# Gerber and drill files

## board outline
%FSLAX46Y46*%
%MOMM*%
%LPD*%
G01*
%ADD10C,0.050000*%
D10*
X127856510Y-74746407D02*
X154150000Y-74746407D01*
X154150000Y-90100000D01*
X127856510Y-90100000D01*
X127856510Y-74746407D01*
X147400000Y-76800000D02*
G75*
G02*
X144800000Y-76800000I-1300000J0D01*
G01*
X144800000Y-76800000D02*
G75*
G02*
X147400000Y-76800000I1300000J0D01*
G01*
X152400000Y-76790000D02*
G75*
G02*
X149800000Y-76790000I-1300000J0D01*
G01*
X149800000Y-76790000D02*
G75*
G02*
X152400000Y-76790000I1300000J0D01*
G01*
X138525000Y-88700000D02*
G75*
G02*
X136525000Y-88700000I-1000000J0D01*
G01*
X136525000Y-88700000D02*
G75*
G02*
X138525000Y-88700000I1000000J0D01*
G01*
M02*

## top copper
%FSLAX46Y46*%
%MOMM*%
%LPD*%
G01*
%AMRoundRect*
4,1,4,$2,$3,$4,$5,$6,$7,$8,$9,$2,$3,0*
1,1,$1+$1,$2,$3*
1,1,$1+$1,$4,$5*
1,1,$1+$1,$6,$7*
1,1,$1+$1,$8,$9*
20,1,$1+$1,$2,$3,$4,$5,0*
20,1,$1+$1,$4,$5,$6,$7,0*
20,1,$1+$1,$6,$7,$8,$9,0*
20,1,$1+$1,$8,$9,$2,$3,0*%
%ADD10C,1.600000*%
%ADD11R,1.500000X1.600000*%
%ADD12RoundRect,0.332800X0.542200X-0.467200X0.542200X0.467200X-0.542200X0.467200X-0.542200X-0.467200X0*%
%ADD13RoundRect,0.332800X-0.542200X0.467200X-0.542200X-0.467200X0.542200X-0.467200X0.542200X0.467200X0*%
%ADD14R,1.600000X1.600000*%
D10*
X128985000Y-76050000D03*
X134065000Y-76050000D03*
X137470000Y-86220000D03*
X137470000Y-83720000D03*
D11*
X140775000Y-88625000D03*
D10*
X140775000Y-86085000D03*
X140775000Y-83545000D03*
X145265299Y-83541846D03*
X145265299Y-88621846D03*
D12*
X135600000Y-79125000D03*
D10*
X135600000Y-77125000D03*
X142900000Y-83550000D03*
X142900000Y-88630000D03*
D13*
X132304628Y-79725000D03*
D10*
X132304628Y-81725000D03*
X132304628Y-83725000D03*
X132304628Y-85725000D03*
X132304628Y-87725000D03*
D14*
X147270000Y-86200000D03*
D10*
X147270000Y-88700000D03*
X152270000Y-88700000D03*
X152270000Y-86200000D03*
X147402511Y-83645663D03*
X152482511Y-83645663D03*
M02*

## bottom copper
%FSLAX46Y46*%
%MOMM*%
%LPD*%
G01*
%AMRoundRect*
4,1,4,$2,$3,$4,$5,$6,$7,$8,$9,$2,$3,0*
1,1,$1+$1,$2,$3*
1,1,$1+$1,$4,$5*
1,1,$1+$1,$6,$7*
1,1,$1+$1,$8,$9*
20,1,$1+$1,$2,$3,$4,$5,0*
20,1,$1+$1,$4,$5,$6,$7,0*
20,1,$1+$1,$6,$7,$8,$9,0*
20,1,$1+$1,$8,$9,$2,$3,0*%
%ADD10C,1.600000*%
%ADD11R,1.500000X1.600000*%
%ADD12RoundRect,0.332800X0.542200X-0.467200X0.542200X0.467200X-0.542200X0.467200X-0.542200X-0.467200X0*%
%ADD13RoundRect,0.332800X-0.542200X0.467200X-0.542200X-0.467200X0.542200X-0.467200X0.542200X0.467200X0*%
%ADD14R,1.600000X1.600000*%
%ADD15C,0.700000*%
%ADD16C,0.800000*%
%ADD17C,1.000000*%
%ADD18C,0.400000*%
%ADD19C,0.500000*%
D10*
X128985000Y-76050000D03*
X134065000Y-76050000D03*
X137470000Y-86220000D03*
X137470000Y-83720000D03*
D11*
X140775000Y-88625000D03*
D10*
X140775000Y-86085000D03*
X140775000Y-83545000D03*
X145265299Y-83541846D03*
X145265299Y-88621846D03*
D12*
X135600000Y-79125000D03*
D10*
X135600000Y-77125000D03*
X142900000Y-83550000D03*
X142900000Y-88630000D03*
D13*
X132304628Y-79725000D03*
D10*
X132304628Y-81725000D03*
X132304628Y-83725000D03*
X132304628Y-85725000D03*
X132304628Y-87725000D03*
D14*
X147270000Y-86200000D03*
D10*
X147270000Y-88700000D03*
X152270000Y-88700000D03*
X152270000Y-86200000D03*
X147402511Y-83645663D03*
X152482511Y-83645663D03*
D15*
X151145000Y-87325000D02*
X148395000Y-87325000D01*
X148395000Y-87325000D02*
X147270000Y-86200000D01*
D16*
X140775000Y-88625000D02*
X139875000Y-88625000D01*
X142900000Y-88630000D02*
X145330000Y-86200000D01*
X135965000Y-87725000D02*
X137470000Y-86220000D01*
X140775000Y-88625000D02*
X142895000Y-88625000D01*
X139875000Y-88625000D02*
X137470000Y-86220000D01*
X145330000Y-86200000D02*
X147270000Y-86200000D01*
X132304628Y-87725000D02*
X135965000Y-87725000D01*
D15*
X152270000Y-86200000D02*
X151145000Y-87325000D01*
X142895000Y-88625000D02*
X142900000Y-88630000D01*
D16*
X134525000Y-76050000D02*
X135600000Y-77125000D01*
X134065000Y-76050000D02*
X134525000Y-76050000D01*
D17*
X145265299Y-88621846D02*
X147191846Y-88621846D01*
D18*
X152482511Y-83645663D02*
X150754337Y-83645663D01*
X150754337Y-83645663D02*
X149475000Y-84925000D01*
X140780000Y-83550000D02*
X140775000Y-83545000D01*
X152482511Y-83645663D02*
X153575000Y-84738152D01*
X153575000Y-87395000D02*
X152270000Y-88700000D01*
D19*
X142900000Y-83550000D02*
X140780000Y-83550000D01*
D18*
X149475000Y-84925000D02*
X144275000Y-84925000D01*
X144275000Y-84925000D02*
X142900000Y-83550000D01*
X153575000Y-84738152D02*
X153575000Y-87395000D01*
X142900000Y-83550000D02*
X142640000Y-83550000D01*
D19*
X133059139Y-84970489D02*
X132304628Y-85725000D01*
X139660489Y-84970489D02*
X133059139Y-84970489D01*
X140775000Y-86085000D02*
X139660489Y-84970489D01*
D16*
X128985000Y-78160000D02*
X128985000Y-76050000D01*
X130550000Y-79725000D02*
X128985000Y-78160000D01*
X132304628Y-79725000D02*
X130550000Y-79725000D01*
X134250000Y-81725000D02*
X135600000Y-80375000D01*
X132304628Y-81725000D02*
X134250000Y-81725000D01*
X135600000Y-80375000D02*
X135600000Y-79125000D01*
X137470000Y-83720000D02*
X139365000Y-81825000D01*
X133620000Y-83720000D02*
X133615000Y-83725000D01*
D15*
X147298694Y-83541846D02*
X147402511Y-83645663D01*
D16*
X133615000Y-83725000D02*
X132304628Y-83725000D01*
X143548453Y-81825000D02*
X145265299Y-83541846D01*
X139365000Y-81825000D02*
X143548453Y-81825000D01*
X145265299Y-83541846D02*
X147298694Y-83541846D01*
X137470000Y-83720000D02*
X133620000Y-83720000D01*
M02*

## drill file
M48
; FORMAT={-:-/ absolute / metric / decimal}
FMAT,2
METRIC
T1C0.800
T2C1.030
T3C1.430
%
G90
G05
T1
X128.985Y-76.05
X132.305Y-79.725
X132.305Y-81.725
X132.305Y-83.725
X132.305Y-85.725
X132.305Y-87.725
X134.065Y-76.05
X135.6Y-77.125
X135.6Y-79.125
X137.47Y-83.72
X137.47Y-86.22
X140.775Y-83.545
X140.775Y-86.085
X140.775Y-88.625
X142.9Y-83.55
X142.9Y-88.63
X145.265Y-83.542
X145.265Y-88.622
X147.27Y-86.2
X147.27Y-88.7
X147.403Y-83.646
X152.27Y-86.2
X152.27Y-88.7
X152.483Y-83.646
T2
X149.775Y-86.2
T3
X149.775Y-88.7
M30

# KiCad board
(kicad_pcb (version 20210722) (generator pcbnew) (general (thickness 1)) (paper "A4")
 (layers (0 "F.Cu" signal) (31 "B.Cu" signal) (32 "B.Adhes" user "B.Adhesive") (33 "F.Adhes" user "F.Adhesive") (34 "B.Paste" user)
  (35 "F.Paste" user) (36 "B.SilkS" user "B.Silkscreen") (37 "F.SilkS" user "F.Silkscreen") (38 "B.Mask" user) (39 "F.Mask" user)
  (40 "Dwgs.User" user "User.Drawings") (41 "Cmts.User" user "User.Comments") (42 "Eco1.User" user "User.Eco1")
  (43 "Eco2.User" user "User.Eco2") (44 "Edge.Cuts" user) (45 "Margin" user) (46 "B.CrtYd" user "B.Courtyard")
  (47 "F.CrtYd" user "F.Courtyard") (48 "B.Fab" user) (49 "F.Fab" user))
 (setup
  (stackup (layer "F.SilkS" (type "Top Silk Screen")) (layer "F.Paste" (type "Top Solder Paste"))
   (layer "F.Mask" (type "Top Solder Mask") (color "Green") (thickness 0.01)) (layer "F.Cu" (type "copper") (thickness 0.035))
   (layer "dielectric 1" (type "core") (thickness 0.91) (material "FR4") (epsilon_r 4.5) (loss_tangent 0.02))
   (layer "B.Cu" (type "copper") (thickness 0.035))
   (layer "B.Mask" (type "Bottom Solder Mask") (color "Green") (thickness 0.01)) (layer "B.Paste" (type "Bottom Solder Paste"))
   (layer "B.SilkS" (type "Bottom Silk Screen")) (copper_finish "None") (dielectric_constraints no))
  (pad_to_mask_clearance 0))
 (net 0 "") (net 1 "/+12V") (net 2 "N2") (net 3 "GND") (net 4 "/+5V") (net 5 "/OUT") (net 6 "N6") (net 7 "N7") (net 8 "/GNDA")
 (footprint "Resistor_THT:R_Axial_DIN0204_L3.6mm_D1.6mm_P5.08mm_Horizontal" (layer "F.Cu") (at 128.985 76.05)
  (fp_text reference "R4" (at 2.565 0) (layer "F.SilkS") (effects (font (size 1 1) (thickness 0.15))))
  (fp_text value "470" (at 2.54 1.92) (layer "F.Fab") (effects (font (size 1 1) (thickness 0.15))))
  (pad "1" thru_hole circle locked (at 0 0) (size 1.6 1.6) (drill 0.8) (layers *.Cu *.Mask) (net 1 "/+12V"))
  (pad "2" thru_hole circle locked (at 5.08 0) (size 1.6 1.6) (drill 0.8) (layers *.Cu *.Mask) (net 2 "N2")))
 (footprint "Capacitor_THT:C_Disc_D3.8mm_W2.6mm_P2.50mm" (layer "F.Cu") (at 137.47 86.22 90)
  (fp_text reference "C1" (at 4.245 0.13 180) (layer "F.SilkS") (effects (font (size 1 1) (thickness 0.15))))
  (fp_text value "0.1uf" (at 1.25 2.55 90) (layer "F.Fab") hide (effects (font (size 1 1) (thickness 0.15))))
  (pad "1" thru_hole circle locked (at 0 0 90) (size 1.6 1.6) (drill 0.8) (layers *.Cu *.Mask) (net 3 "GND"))
  (pad "2" thru_hole circle locked (at 2.5 0 90) (size 1.6 1.6) (drill 0.8) (layers *.Cu *.Mask) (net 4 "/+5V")))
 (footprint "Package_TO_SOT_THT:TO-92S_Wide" (layer "F.Cu") (at 140.775 88.625 90)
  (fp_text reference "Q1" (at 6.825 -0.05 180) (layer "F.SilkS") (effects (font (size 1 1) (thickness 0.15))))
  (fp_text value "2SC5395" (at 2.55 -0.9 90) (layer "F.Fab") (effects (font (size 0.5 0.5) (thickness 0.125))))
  (pad "1" thru_hole rect locked (at 0 0 90) (size 1.6 1.5) (drill 0.8) (layers *.Cu *.Mask) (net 3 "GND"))
  (pad "2" thru_hole circle locked (at 2.54 0 90) (size 1.6 1.6) (drill 0.8) (layers *.Cu *.Mask) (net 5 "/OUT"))
  (pad "3" thru_hole circle locked (at 5.08 0 90) (size 1.6 1.6) (drill 0.8) (layers *.Cu *.Mask) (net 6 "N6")))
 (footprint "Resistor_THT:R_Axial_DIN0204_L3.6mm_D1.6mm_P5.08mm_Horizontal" (layer "F.Cu") (at 145.265299 83.541846 -90)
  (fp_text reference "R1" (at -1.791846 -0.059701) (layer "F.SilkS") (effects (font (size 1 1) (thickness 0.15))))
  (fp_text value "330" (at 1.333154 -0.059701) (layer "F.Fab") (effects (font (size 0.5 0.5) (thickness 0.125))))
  (pad "1" thru_hole circle locked (at 0 0 270) (size 1.6 1.6) (drill 0.8) (layers *.Cu *.Mask) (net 4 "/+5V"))
  (pad "2" thru_hole circle locked (at 5.08 0 270) (size 1.6 1.6) (drill 0.8) (layers *.Cu *.Mask) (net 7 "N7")))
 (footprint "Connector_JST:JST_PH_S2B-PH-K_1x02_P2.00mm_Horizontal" (layer "F.Cu") (at 135.6 79.125 90)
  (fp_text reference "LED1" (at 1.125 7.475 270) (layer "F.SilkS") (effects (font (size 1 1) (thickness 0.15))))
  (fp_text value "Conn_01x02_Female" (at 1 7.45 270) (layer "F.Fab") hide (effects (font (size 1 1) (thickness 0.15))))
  (pad "1" thru_hole roundrect locked (at 0 0 90) (size 1.6 1.75) (drill 0.8) (layers *.Cu *.Mask) (roundrect_rratio 0.208) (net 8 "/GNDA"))
  (pad "2" thru_hole circle locked (at 2 0 90) (size 1.6 1.6) (drill 0.8) (layers *.Cu *.Mask) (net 2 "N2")))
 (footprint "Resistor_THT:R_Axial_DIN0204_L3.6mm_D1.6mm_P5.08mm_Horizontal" (layer "F.Cu") (at 142.9 83.55 -90)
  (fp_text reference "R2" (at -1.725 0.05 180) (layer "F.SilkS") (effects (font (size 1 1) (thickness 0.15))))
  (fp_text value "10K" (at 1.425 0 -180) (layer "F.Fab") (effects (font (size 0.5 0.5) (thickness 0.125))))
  (pad "1" thru_hole circle locked (at 0 0 270) (size 1.6 1.6) (drill 0.8) (layers *.Cu *.Mask) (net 6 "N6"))
  (pad "2" thru_hole circle locked (at 5.08 0 270) (size 1.6 1.6) (drill 0.8) (layers *.Cu *.Mask) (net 3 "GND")))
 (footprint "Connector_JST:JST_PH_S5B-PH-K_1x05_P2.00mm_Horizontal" (layer "F.Cu") (at 132.304628 79.725 -90)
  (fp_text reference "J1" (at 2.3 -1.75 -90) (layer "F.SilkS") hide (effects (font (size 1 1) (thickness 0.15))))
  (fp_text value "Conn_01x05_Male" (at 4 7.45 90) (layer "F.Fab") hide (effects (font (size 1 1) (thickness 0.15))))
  (pad "1" thru_hole roundrect locked (at 0 0 270) (size 1.6 1.75) (drill 0.8) (layers *.Cu *.Mask) (roundrect_rratio 0.208) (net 1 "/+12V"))
  (pad "2" thru_hole circle locked (at 2 0 270) (size 1.6 1.6) (drill 0.8) (layers *.Cu *.Mask) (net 8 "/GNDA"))
  (pad "3" thru_hole circle locked (at 4 0 270) (size 1.6 1.6) (drill 0.8) (layers *.Cu *.Mask) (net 4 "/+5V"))
  (pad "4" thru_hole circle locked (at 6 0 270) (size 1.6 1.6) (drill 0.8) (layers *.Cu *.Mask) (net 5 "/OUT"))
  (pad "5" thru_hole circle locked (at 8 0 270) (size 1.6 1.6) (drill 0.8) (layers *.Cu *.Mask) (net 3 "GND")))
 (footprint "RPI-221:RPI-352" (layer "F.Cu") (at 146.5 89.6)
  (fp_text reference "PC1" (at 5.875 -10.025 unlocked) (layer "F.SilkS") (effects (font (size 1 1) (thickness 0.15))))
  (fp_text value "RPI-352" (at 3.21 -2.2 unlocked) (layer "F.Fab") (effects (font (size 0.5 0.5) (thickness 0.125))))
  (pad "" np_thru_hole circle locked (at 3.275 -3.4) (size 1.03 1.03) (drill 1.03) (layers *.Mask))
  (pad "" np_thru_hole circle locked (at 3.275 -0.9) (size 1.43 1.43) (drill 1.43) (layers *.Mask))
  (pad "1" thru_hole rect locked (at 0.77 -3.4) (size 1.6 1.6) (drill oval 0.8) (layers *.Cu *.Mask) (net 3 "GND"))
  (pad "2" thru_hole circle locked (at 0.77 -0.9) (size 1.6 1.6) (drill oval 0.8) (layers *.Cu *.Mask) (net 7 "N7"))
  (pad "3" thru_hole circle locked (at 5.77 -0.9) (size 1.6 1.6) (drill oval 0.8) (layers *.Cu *.Mask) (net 6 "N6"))
  (pad "4" thru_hole circle locked (at 5.77 -3.4) (size 1.6 1.6) (drill oval 0.8) (layers *.Cu *.Mask) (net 3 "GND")))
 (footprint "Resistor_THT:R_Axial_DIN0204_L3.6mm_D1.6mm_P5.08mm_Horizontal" (layer "F.Cu") (at 147.402511 83.645663)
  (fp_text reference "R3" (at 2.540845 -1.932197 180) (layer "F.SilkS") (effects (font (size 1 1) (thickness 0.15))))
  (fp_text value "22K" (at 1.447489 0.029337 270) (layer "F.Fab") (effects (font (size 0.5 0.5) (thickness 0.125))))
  (pad "1" thru_hole circle locked (at 0 0) (size 1.6 1.6) (drill 0.8) (layers *.Cu *.Mask) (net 4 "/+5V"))
  (pad "2" thru_hole circle locked (at 5.08 0) (size 1.6 1.6) (drill 0.8) (layers *.Cu *.Mask) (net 6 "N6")))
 (gr_rect (start 127.85651 74.746407) (end 154.15 90.1) (layer "Edge.Cuts") (width 0.05) (fill none))
 (gr_circle (center 146.1 76.8) (end 147.4 76.8) (layer "Edge.Cuts") (width 0.05) (fill none))
 (gr_circle (center 151.1 76.79) (end 152.4 76.79) (layer "Edge.Cuts") (width 0.05) (fill none))
 (gr_circle (center 137.525 88.7) (end 138.525 88.7) (layer "Edge.Cuts") (width 0.05) (fill none))
 (segment (start 151.145 87.325) (end 148.395 87.325) (width 0.7) (layer "B.Cu") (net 3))
 (segment (start 148.395 87.325) (end 147.27 86.2) (width 0.7) (layer "B.Cu") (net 3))
 (segment (start 140.775 88.625) (end 139.875 88.625) (width 0.8) (layer "B.Cu") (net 3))
 (segment (start 142.9 88.63) (end 145.33 86.2) (width 0.8) (layer "B.Cu") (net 3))
 (segment (start 135.965 87.725) (end 137.47 86.22) (width 0.8) (layer "B.Cu") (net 3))
 (segment (start 140.775 88.625) (end 142.895 88.625) (width 0.8) (layer "B.Cu") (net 3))
 (segment (start 139.875 88.625) (end 137.47 86.22) (width 0.8) (layer "B.Cu") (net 3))
 (segment (start 145.33 86.2) (end 147.27 86.2) (width 0.8) (layer "B.Cu") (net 3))
 (segment (start 132.304628 87.725) (end 135.965 87.725) (width 0.8) (layer "B.Cu") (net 3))
 (segment (start 152.27 86.2) (end 151.145 87.325) (width 0.7) (layer "B.Cu") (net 3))
 (segment (start 142.895 88.625) (end 142.9 88.63) (width 0.7) (layer "B.Cu") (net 3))
 (segment (start 134.525 76.05) (end 135.6 77.125) (width 0.8) (layer "B.Cu") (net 2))
 (segment (start 134.065 76.05) (end 134.525 76.05) (width 0.8) (layer "B.Cu") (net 2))
 (segment (start 145.265299 88.621846) (end 147.191846 88.621846) (width 1) (layer "B.Cu") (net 7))
 (segment (start 152.482511 83.645663) (end 150.754337 83.645663) (width 0.4) (layer "B.Cu") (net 6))
 (segment (start 150.754337 83.645663) (end 149.475 84.925) (width 0.4) (layer "B.Cu") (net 6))
 (segment (start 140.78 83.55) (end 140.775 83.545) (width 0.4) (layer "B.Cu") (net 6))
 (segment (start 152.482511 83.645663) (end 153.575 84.738152) (width 0.4) (layer "B.Cu") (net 6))
 (segment (start 153.575 87.395) (end 152.27 88.7) (width 0.4) (layer "B.Cu") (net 6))
 (segment (start 142.9 83.55) (end 140.78 83.55) (width 0.5) (layer "B.Cu") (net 6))
 (segment (start 149.475 84.925) (end 144.275 84.925) (width 0.4) (layer "B.Cu") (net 6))
 (segment (start 144.275 84.925) (end 142.9 83.55) (width 0.4) (layer "B.Cu") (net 6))
 (segment (start 153.575 84.738152) (end 153.575 87.395) (width 0.4) (layer "B.Cu") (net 6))
 (segment (start 142.9 83.55) (end 142.64 83.55) (width 0.4) (layer "B.Cu") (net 6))
 (segment (start 133.059139 84.970489) (end 132.304628 85.725) (width 0.5) (layer "B.Cu") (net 5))
 (segment (start 139.660489 84.970489) (end 133.059139 84.970489) (width 0.5) (layer "B.Cu") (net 5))
 (segment (start 140.775 86.085) (end 139.660489 84.970489) (width 0.5) (layer "B.Cu") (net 5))
 (segment (start 128.985 78.16) (end 128.985 76.05) (width 0.8) (layer "B.Cu") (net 1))
 (segment (start 130.55 79.725) (end 128.985 78.16) (width 0.8) (layer "B.Cu") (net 1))
 (segment (start 132.304628 79.725) (end 130.55 79.725) (width 0.8) (layer "B.Cu") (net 1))
 (segment (start 134.25 81.725) (end 135.6 80.375) (width 0.8) (layer "B.Cu") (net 8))
 (segment (start 132.304628 81.725) (end 134.25 81.725) (width 0.8) (layer "B.Cu") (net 8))
 (segment (start 135.6 80.375) (end 135.6 79.125) (width 0.8) (layer "B.Cu") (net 8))
 (segment (start 137.47 83.72) (end 139.365 81.825) (width 0.8) (layer "B.Cu") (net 4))
 (segment (start 133.62 83.72) (end 133.615 83.725) (width 0.8) (layer "B.Cu") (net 4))
 (segment (start 147.298694 83.541846) (end 147.402511 83.645663) (width 0.7) (layer "B.Cu") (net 4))
 (segment (start 133.615 83.725) (end 132.304628 83.725) (width 0.8) (layer "B.Cu") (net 4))
 (segment (start 143.548453 81.825) (end 145.265299 83.541846) (width 0.8) (layer "B.Cu") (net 4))
 (segment (start 139.365 81.825) (end 143.548453 81.825) (width 0.8) (layer "B.Cu") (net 4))
 (segment (start 145.265299 83.541846) (end 147.298694 83.541846) (width 0.8) (layer "B.Cu") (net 4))
 (segment (start 137.47 83.72) (end 133.62 83.72) (width 0.8) (layer "B.Cu") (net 4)))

